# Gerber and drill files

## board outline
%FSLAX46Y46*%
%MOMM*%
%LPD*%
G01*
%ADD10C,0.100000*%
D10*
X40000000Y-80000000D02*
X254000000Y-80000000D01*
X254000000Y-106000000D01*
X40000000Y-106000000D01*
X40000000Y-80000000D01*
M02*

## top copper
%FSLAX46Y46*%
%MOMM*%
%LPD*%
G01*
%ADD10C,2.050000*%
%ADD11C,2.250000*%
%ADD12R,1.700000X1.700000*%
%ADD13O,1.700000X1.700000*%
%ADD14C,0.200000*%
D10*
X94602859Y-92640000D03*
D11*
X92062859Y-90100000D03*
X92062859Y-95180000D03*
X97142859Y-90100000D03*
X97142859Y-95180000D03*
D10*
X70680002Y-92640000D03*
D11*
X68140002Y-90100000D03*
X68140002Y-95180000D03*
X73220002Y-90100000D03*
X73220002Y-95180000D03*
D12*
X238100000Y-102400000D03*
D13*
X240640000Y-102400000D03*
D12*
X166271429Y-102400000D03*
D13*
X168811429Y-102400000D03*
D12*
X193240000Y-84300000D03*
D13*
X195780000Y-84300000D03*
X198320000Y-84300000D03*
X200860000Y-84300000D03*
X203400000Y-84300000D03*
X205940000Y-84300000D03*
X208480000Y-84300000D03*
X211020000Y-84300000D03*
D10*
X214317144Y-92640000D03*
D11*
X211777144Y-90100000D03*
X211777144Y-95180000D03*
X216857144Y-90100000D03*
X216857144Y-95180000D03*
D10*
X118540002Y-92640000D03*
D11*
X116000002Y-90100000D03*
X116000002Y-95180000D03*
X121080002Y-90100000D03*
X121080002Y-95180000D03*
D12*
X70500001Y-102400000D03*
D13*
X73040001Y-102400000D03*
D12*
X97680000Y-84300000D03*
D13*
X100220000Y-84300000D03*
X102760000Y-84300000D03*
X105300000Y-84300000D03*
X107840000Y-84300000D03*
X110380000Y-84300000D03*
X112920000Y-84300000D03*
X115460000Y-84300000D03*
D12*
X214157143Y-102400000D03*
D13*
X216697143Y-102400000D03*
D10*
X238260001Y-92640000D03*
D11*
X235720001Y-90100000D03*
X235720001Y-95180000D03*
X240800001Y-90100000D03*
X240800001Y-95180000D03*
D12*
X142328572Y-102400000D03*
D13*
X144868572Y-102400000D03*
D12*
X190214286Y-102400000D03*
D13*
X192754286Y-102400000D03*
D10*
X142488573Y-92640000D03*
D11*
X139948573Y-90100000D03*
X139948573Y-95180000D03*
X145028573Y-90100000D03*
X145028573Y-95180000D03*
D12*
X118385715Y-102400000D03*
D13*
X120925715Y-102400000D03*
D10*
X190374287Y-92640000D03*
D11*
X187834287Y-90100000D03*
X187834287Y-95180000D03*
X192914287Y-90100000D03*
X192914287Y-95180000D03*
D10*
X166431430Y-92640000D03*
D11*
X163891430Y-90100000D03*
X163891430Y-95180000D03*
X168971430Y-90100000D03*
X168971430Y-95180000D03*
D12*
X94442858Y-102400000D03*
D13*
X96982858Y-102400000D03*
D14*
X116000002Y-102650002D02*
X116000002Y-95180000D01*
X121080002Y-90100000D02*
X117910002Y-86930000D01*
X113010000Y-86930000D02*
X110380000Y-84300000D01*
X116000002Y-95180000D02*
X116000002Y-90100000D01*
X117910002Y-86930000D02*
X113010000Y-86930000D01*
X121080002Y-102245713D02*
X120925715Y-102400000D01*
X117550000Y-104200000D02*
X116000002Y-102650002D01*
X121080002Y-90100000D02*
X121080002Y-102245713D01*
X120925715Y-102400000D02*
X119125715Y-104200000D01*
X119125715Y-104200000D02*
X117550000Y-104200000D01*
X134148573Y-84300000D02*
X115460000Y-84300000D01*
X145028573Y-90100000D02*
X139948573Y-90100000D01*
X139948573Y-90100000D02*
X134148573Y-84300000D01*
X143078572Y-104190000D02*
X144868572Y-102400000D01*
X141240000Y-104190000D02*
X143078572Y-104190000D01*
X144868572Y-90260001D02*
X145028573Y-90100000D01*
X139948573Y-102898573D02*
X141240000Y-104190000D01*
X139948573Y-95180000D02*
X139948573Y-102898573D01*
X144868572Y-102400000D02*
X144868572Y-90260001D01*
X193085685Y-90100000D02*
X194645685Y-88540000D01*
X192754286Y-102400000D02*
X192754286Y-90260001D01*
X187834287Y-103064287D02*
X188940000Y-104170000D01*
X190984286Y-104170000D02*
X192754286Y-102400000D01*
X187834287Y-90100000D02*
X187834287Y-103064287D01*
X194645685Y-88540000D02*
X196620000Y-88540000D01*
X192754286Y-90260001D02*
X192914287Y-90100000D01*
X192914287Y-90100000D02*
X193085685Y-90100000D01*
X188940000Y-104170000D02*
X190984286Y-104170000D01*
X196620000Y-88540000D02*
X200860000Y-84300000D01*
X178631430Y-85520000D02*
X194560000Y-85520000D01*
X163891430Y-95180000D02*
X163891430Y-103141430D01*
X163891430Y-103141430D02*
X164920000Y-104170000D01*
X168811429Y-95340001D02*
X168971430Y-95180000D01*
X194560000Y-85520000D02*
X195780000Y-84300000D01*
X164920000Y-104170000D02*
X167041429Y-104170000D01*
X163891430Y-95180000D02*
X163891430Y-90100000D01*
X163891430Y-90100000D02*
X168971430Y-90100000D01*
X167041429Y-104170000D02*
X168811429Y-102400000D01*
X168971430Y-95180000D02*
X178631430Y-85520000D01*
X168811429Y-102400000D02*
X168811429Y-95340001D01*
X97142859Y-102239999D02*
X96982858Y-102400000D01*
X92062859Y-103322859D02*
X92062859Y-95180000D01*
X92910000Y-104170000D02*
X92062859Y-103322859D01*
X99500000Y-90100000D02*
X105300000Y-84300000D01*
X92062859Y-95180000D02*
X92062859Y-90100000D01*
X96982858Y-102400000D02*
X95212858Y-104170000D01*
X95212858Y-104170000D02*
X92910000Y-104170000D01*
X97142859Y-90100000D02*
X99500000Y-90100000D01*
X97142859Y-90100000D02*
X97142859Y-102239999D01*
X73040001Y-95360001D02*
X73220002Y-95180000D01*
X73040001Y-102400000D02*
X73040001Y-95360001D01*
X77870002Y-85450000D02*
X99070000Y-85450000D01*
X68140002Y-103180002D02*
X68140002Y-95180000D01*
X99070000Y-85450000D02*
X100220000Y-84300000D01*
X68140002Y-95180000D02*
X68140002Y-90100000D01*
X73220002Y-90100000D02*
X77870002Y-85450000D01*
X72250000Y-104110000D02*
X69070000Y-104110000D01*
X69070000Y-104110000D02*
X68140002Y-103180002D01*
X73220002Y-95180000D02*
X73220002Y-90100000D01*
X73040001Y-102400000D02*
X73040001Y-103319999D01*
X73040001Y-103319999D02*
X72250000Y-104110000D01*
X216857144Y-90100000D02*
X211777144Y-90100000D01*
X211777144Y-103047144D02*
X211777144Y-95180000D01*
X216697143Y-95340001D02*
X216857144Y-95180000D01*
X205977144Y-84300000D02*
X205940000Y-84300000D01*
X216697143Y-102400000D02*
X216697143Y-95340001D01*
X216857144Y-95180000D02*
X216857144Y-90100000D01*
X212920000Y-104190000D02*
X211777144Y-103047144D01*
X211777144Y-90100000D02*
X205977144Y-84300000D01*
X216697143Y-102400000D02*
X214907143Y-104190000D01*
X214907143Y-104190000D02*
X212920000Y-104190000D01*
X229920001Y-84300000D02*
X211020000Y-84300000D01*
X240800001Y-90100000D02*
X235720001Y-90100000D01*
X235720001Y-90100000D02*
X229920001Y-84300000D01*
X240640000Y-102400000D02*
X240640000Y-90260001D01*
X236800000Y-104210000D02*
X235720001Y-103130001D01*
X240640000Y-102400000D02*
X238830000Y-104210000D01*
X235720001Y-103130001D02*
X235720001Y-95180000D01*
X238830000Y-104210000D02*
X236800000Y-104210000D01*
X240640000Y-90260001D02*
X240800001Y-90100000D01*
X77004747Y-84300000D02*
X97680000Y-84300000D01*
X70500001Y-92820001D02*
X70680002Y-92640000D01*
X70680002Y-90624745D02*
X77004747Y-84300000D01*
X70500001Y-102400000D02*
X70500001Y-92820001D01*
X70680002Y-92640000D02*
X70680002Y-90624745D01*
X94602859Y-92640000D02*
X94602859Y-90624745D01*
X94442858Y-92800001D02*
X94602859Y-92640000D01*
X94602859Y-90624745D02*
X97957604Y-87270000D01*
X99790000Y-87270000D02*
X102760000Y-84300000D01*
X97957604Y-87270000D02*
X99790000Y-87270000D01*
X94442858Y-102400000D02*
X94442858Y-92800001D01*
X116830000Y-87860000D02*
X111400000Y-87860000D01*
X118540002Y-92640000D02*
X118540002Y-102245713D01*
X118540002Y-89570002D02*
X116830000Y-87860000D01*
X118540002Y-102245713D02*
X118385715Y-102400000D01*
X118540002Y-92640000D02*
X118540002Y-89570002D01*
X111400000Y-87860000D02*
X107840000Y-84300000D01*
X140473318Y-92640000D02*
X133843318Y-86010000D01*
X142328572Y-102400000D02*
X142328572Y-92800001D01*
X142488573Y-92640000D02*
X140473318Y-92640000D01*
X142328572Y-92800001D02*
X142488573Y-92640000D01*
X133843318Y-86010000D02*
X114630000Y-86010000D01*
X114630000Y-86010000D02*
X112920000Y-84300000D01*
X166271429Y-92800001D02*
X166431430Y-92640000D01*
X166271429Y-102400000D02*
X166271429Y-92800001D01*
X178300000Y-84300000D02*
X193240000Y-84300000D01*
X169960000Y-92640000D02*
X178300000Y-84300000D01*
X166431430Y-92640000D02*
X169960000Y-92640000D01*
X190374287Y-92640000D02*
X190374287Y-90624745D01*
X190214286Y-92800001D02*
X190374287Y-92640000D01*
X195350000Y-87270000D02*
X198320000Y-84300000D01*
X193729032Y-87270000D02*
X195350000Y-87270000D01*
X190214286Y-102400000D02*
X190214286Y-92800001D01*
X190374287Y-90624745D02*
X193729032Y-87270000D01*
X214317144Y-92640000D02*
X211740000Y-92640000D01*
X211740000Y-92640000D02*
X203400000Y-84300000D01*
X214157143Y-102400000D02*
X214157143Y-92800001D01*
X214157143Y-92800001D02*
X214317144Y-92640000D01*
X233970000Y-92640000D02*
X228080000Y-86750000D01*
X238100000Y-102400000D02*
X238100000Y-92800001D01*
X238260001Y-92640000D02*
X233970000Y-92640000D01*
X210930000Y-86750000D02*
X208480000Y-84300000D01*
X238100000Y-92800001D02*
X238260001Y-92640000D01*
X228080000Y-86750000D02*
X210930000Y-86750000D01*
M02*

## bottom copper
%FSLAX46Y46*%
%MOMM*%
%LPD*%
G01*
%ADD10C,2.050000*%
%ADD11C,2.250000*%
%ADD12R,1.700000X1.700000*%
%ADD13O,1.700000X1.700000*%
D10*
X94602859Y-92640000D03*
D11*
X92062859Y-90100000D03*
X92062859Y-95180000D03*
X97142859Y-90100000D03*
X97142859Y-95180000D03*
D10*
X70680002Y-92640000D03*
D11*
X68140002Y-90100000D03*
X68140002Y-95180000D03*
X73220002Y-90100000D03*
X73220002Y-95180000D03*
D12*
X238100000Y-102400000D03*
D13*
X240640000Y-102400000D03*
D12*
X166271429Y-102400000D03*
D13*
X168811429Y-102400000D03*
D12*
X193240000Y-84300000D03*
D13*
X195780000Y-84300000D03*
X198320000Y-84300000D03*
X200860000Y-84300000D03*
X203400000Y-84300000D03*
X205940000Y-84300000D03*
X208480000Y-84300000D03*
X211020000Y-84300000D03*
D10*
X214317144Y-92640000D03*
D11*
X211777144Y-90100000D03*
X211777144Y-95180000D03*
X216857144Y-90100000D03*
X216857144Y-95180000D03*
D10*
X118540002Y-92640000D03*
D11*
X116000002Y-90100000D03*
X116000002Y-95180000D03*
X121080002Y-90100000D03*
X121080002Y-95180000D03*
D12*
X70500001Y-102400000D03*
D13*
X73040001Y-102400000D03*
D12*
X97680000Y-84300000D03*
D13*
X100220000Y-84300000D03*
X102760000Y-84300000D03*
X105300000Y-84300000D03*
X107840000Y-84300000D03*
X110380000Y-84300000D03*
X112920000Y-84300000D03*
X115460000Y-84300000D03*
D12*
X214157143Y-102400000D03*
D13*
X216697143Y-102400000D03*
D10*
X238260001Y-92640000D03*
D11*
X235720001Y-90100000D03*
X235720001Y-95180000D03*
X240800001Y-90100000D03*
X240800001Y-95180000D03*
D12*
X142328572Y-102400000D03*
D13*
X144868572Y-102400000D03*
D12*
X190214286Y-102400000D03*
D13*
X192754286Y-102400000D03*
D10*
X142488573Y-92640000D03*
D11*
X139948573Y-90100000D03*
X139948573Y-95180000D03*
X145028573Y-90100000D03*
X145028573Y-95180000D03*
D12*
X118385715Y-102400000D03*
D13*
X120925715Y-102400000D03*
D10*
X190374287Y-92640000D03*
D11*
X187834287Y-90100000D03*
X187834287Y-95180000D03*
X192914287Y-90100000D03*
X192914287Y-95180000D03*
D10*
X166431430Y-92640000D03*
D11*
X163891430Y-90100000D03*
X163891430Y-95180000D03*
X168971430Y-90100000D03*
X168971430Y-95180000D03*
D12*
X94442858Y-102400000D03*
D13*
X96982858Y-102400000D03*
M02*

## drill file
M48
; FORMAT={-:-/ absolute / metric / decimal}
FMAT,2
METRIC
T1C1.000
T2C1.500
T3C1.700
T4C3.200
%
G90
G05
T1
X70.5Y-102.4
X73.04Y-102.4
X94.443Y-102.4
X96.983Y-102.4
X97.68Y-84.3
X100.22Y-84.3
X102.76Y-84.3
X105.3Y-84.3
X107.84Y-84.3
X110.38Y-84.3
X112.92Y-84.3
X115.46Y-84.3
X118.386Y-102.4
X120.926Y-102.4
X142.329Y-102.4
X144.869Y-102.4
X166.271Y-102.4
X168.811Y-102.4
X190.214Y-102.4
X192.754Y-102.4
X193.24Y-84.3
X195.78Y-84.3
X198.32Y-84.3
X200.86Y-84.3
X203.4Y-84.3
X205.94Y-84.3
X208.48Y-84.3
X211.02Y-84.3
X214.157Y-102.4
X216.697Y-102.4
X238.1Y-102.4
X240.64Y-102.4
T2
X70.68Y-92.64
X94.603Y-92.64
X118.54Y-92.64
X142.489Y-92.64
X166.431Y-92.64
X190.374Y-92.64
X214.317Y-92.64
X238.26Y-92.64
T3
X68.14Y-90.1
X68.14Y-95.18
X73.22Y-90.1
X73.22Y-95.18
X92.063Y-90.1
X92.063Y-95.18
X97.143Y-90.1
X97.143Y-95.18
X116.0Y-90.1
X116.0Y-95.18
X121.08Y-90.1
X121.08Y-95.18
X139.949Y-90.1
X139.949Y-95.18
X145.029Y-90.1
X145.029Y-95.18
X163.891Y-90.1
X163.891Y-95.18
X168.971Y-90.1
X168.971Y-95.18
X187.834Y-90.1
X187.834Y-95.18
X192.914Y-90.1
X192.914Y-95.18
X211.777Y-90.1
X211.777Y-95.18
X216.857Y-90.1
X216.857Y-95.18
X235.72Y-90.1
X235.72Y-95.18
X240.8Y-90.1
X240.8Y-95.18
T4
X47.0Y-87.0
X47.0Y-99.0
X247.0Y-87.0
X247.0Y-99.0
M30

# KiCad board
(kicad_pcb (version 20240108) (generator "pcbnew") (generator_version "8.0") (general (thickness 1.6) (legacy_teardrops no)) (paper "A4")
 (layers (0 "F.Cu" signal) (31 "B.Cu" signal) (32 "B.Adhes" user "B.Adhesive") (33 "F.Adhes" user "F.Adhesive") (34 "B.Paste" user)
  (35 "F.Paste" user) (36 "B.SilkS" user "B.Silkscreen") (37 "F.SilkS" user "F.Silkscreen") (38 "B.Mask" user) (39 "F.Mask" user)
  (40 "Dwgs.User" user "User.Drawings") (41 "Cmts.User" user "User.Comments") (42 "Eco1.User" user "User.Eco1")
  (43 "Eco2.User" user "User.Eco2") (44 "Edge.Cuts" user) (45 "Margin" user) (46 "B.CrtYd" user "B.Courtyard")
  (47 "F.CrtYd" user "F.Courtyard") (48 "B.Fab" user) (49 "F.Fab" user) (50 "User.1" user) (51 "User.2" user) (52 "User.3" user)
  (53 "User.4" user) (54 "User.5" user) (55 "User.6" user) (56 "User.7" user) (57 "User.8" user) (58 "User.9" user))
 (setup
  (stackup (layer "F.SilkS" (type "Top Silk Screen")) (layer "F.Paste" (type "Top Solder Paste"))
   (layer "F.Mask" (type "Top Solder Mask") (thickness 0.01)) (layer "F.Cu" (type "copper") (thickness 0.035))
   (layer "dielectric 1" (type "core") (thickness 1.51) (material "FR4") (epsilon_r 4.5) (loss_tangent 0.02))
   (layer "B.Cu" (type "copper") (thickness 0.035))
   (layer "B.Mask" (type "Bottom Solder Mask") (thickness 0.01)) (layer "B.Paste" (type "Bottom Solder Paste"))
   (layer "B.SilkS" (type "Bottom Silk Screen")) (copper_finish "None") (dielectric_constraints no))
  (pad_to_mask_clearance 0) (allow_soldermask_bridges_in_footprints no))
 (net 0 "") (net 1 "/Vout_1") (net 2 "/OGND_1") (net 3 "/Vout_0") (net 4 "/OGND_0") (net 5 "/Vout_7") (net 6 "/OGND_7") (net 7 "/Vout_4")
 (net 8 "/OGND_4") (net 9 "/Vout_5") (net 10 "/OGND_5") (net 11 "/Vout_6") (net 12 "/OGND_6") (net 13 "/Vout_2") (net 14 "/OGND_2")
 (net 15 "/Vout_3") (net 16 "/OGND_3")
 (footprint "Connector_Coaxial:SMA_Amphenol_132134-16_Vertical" (layer "F.Cu") (at 94.602859 92.64)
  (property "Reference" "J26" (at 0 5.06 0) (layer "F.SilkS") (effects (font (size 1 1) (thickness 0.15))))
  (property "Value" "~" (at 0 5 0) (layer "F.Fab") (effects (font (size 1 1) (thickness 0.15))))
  (pad "1" thru_hole circle (at 0 0) (size 2.05 2.05) (drill 1.5) (layers "*.Cu" "*.Mask") (remove_unused_layers no) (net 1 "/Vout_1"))
  (pad "2" thru_hole circle (at -2.54 -2.54) (size 2.25 2.25) (drill 1.7) (layers "*.Cu" "*.Mask") (remove_unused_layers no)
   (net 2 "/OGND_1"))
  (pad "2" thru_hole circle (at -2.54 2.54) (size 2.25 2.25) (drill 1.7) (layers "*.Cu" "*.Mask") (remove_unused_layers no)
   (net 2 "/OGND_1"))
  (pad "2" thru_hole circle (at 2.54 -2.54) (size 2.25 2.25) (drill 1.7) (layers "*.Cu" "*.Mask") (remove_unused_layers no)
   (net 2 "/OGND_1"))
  (pad "2" thru_hole circle (at 2.54 2.54) (size 2.25 2.25) (drill 1.7) (layers "*.Cu" "*.Mask") (remove_unused_layers no) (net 2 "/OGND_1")))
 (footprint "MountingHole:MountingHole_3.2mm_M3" (layer "F.Cu") (at 247 99)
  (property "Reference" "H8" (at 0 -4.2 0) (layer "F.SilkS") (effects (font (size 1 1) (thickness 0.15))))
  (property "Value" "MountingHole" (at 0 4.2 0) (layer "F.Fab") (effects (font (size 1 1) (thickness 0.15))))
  (pad "" np_thru_hole circle (at 0 0) (size 3.2 3.2) (drill 3.2) (layers "*.Cu" "*.Mask")))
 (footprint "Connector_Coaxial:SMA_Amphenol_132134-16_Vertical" (layer "F.Cu") (at 70.680002 92.64)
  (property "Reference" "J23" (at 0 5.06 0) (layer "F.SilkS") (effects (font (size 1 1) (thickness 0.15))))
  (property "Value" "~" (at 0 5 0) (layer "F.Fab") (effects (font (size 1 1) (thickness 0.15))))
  (pad "1" thru_hole circle (at 0 0) (size 2.05 2.05) (drill 1.5) (layers "*.Cu" "*.Mask") (remove_unused_layers no) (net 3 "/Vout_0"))
  (pad "2" thru_hole circle (at -2.54 -2.54) (size 2.25 2.25) (drill 1.7) (layers "*.Cu" "*.Mask") (remove_unused_layers no)
   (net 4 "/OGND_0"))
  (pad "2" thru_hole circle (at -2.54 2.54) (size 2.25 2.25) (drill 1.7) (layers "*.Cu" "*.Mask") (remove_unused_layers no)
   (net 4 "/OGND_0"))
  (pad "2" thru_hole circle (at 2.54 -2.54) (size 2.25 2.25) (drill 1.7) (layers "*.Cu" "*.Mask") (remove_unused_layers no)
   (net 4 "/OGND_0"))
  (pad "2" thru_hole circle (at 2.54 2.54) (size 2.25 2.25) (drill 1.7) (layers "*.Cu" "*.Mask") (remove_unused_layers no) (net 4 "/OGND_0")))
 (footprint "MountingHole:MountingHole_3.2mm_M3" (layer "F.Cu") (at 47 99)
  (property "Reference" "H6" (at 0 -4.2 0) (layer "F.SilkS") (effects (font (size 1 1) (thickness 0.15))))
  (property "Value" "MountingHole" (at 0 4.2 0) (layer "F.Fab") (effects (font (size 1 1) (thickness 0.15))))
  (pad "" np_thru_hole circle (at 0 0) (size 3.2 3.2) (drill 3.2) (layers "*.Cu" "*.Mask")))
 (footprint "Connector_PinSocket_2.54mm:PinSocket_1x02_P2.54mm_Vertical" (layer "F.Cu") (at 238.1 102.4 90)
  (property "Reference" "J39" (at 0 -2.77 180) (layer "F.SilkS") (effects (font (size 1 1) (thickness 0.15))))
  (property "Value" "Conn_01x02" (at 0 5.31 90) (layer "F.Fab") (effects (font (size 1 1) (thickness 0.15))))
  (pad "1" thru_hole rect (at 0 0 90) (size 1.7 1.7) (drill 1) (layers "*.Cu" "*.Mask") (remove_unused_layers no) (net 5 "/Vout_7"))
  (pad "2" thru_hole oval (at 0 2.54 90) (size 1.7 1.7) (drill 1) (layers "*.Cu" "*.Mask") (remove_unused_layers no) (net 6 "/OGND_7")))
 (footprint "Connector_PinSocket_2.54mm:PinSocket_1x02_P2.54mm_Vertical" (layer "F.Cu") (at 166.271429 102.4 90)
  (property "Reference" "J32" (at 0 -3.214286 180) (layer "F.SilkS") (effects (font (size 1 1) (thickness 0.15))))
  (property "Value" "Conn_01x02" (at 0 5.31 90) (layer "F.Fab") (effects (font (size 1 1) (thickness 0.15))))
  (pad "1" thru_hole rect (at 0 0 90) (size 1.7 1.7) (drill 1) (layers "*.Cu" "*.Mask") (remove_unused_layers no) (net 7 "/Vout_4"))
  (pad "2" thru_hole oval (at 0 2.54 90) (size 1.7 1.7) (drill 1) (layers "*.Cu" "*.Mask") (remove_unused_layers no) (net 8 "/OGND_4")))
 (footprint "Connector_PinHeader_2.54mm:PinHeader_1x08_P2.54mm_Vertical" (layer "F.Cu") (at 193.24 84.3 90)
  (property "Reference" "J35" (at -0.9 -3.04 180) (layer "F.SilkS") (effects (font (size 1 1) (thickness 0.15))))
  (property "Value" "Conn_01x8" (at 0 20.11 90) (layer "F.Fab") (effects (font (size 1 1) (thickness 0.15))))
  (pad "1" thru_hole rect (at 0 0 90) (size 1.7 1.7) (drill 1) (layers "*.Cu" "*.Mask") (remove_unused_layers no) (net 7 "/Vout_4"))
  (pad "2" thru_hole oval (at 0 2.54 90) (size 1.7 1.7) (drill 1) (layers "*.Cu" "*.Mask") (remove_unused_layers no) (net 8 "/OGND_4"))
  (pad "3" thru_hole oval (at 0 5.08 90) (size 1.7 1.7) (drill 1) (layers "*.Cu" "*.Mask") (remove_unused_layers no) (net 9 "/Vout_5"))
  (pad "4" thru_hole oval (at 0 7.62 90) (size 1.7 1.7) (drill 1) (layers "*.Cu" "*.Mask") (remove_unused_layers no) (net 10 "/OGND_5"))
  (pad "5" thru_hole oval (at 0 10.16 90) (size 1.7 1.7) (drill 1) (layers "*.Cu" "*.Mask") (remove_unused_layers no) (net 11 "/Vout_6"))
  (pad "6" thru_hole oval (at 0 12.7 90) (size 1.7 1.7) (drill 1) (layers "*.Cu" "*.Mask") (remove_unused_layers no) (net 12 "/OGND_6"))
  (pad "7" thru_hole oval (at 0 15.24 90) (size 1.7 1.7) (drill 1) (layers "*.Cu" "*.Mask") (remove_unused_layers no) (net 5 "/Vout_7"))
  (pad "8" thru_hole oval (at 0 17.78 90) (size 1.7 1.7) (drill 1) (layers "*.Cu" "*.Mask") (remove_unused_layers no) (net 6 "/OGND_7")))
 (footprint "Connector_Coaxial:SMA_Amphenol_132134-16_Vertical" (layer "F.Cu") (at 214.317144 92.64)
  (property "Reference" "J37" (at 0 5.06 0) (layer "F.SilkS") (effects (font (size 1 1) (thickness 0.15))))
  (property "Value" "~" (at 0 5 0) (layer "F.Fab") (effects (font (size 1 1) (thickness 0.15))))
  (pad "1" thru_hole circle (at 0 0) (size 2.05 2.05) (drill 1.5) (layers "*.Cu" "*.Mask") (remove_unused_layers no) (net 11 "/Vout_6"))
  (pad "2" thru_hole circle (at -2.54 -2.54) (size 2.25 2.25) (drill 1.7) (layers "*.Cu" "*.Mask") (remove_unused_layers no)
   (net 12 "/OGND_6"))
  (pad "2" thru_hole circle (at -2.54 2.54) (size 2.25 2.25) (drill 1.7) (layers "*.Cu" "*.Mask") (remove_unused_layers no)
   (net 12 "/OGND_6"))
  (pad "2" thru_hole circle (at 2.54 -2.54) (size 2.25 2.25) (drill 1.7) (layers "*.Cu" "*.Mask") (remove_unused_layers no)
   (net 12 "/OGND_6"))
  (pad "2" thru_hole circle (at 2.54 2.54) (size 2.25 2.25) (drill 1.7) (layers "*.Cu" "*.Mask") (remove_unused_layers no)
   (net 12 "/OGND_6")))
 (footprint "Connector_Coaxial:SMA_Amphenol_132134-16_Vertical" (layer "F.Cu") (at 118.540002 92.64)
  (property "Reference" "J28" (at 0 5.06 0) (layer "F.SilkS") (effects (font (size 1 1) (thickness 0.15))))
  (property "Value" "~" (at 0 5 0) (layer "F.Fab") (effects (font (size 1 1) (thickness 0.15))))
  (pad "1" thru_hole circle (at 0 0) (size 2.05 2.05) (drill 1.5) (layers "*.Cu" "*.Mask") (remove_unused_layers no) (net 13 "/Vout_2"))
  (pad "2" thru_hole circle (at -2.54 -2.54) (size 2.25 2.25) (drill 1.7) (layers "*.Cu" "*.Mask") (remove_unused_layers no)
   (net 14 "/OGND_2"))
  (pad "2" thru_hole circle (at -2.54 2.54) (size 2.25 2.25) (drill 1.7) (layers "*.Cu" "*.Mask") (remove_unused_layers no)
   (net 14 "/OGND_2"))
  (pad "2" thru_hole circle (at 2.54 -2.54) (size 2.25 2.25) (drill 1.7) (layers "*.Cu" "*.Mask") (remove_unused_layers no)
   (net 14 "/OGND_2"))
  (pad "2" thru_hole circle (at 2.54 2.54) (size 2.25 2.25) (drill 1.7) (layers "*.Cu" "*.Mask") (remove_unused_layers no)
   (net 14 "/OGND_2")))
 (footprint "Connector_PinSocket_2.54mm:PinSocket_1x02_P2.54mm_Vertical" (layer "F.Cu") (at 70.500001 102.4 90)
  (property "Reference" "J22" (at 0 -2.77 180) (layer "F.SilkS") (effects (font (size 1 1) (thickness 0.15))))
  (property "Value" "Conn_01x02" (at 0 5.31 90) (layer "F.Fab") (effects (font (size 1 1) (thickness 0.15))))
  (pad "1" thru_hole rect (at 0 0 90) (size 1.7 1.7) (drill 1) (layers "*.Cu" "*.Mask") (remove_unused_layers no) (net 3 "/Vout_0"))
  (pad "2" thru_hole oval (at 0 2.54 90) (size 1.7 1.7) (drill 1) (layers "*.Cu" "*.Mask") (remove_unused_layers no) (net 4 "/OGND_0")))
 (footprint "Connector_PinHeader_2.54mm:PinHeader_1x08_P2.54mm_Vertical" (layer "F.Cu") (at 97.68 84.3 90)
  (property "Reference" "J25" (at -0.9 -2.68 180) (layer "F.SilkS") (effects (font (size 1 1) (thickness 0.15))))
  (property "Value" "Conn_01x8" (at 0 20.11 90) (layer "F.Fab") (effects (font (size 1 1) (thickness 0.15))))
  (pad "1" thru_hole rect (at 0 0 90) (size 1.7 1.7) (drill 1) (layers "*.Cu" "*.Mask") (remove_unused_layers no) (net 3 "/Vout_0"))
  (pad "2" thru_hole oval (at 0 2.54 90) (size 1.7 1.7) (drill 1) (layers "*.Cu" "*.Mask") (remove_unused_layers no) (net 4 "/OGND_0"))
  (pad "3" thru_hole oval (at 0 5.08 90) (size 1.7 1.7) (drill 1) (layers "*.Cu" "*.Mask") (remove_unused_layers no) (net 1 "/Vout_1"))
  (pad "4" thru_hole oval (at 0 7.62 90) (size 1.7 1.7) (drill 1) (layers "*.Cu" "*.Mask") (remove_unused_layers no) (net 2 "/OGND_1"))
  (pad "5" thru_hole oval (at 0 10.16 90) (size 1.7 1.7) (drill 1) (layers "*.Cu" "*.Mask") (remove_unused_layers no) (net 13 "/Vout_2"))
  (pad "6" thru_hole oval (at 0 12.7 90) (size 1.7 1.7) (drill 1) (layers "*.Cu" "*.Mask") (remove_unused_layers no) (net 14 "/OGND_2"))
  (pad "7" thru_hole oval (at 0 15.24 90) (size 1.7 1.7) (drill 1) (layers "*.Cu" "*.Mask") (remove_unused_layers no) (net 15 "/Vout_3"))
  (pad "8" thru_hole oval (at 0 17.78 90) (size 1.7 1.7) (drill 1) (layers "*.Cu" "*.Mask") (remove_unused_layers no) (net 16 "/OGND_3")))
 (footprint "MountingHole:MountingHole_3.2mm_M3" (layer "F.Cu") (at 247 87)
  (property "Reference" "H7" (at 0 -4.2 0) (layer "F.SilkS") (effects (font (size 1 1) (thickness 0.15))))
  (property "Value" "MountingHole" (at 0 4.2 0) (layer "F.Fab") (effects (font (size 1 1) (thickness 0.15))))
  (pad "" np_thru_hole circle (at 0 0) (size 3.2 3.2) (drill 3.2) (layers "*.Cu" "*.Mask")))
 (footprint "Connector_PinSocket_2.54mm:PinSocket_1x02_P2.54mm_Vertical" (layer "F.Cu") (at 214.157143 102.4 90)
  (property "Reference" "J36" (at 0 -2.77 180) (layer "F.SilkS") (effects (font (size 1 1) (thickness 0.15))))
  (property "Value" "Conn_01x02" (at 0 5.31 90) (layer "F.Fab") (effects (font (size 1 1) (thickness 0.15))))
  (pad "1" thru_hole rect (at 0 0 90) (size 1.7 1.7) (drill 1) (layers "*.Cu" "*.Mask") (remove_unused_layers no) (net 11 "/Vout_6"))
  (pad "2" thru_hole oval (at 0 2.54 90) (size 1.7 1.7) (drill 1) (layers "*.Cu" "*.Mask") (remove_unused_layers no) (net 12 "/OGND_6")))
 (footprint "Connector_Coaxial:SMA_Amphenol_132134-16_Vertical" (layer "F.Cu") (at 238.260001 92.64)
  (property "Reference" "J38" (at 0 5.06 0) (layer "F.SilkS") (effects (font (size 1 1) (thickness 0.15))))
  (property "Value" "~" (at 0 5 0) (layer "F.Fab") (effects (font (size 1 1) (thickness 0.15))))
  (pad "1" thru_hole circle (at 0 0) (size 2.05 2.05) (drill 1.5) (layers "*.Cu" "*.Mask") (remove_unused_layers no) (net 5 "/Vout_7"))
  (pad "2" thru_hole circle (at -2.54 -2.54) (size 2.25 2.25) (drill 1.7) (layers "*.Cu" "*.Mask") (remove_unused_layers no)
   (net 6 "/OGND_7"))
  (pad "2" thru_hole circle (at -2.54 2.54) (size 2.25 2.25) (drill 1.7) (layers "*.Cu" "*.Mask") (remove_unused_layers no)
   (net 6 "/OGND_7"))
  (pad "2" thru_hole circle (at 2.54 -2.54) (size 2.25 2.25) (drill 1.7) (layers "*.Cu" "*.Mask") (remove_unused_layers no)
   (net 6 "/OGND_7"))
  (pad "2" thru_hole circle (at 2.54 2.54) (size 2.25 2.25) (drill 1.7) (layers "*.Cu" "*.Mask") (remove_unused_layers no) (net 6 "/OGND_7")))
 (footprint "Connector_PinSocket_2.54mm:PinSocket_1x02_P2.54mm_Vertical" (layer "F.Cu") (at 142.328572 102.4 90)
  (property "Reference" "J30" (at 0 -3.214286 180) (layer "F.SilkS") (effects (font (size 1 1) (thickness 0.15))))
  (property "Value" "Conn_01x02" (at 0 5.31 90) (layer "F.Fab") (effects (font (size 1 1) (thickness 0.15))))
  (pad "1" thru_hole rect (at 0 0 90) (size 1.7 1.7) (drill 1) (layers "*.Cu" "*.Mask") (remove_unused_layers no) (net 15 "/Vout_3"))
  (pad "2" thru_hole oval (at 0 2.54 90) (size 1.7 1.7) (drill 1) (layers "*.Cu" "*.Mask") (remove_unused_layers no) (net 16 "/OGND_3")))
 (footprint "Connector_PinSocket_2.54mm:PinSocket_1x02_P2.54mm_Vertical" (layer "F.Cu") (at 190.214286 102.4 90)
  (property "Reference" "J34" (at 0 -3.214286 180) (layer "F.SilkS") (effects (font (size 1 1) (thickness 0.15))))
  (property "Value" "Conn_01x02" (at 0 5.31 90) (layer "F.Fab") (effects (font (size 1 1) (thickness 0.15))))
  (pad "1" thru_hole rect (at 0 0 90) (size 1.7 1.7) (drill 1) (layers "*.Cu" "*.Mask") (remove_unused_layers no) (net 9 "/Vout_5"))
  (pad "2" thru_hole oval (at 0 2.54 90) (size 1.7 1.7) (drill 1) (layers "*.Cu" "*.Mask") (remove_unused_layers no) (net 10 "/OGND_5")))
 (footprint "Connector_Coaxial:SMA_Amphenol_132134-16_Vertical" (layer "F.Cu") (at 142.488573 92.64)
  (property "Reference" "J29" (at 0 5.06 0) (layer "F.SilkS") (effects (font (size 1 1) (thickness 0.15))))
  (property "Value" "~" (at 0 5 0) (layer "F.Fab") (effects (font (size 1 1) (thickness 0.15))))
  (pad "1" thru_hole circle (at 0 0) (size 2.05 2.05) (drill 1.5) (layers "*.Cu" "*.Mask") (remove_unused_layers no) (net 15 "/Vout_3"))
  (pad "2" thru_hole circle (at -2.54 -2.54) (size 2.25 2.25) (drill 1.7) (layers "*.Cu" "*.Mask") (remove_unused_layers no)
   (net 16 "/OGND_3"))
  (pad "2" thru_hole circle (at -2.54 2.54) (size 2.25 2.25) (drill 1.7) (layers "*.Cu" "*.Mask") (remove_unused_layers no)
   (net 16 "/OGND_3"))
  (pad "2" thru_hole circle (at 2.54 -2.54) (size 2.25 2.25) (drill 1.7) (layers "*.Cu" "*.Mask") (remove_unused_layers no)
   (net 16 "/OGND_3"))
  (pad "2" thru_hole circle (at 2.54 2.54) (size 2.25 2.25) (drill 1.7) (layers "*.Cu" "*.Mask") (remove_unused_layers no)
   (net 16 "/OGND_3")))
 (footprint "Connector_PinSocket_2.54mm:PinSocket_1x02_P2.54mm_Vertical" (layer "F.Cu") (at 118.385715 102.4 90)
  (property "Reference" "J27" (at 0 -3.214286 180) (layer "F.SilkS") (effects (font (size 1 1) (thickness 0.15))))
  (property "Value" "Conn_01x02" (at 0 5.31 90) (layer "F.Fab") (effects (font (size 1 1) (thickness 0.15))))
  (pad "1" thru_hole rect (at 0 0 90) (size 1.7 1.7) (drill 1) (layers "*.Cu" "*.Mask") (remove_unused_layers no) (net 13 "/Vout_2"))
  (pad "2" thru_hole oval (at 0 2.54 90) (size 1.7 1.7) (drill 1) (layers "*.Cu" "*.Mask") (remove_unused_layers no) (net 14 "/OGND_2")))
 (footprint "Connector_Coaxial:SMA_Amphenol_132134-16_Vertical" (layer "F.Cu") (at 190.374287 92.64)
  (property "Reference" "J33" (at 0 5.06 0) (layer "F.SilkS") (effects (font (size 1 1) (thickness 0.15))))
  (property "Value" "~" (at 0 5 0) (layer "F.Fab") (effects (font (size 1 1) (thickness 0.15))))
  (pad "1" thru_hole circle (at 0 0) (size 2.05 2.05) (drill 1.5) (layers "*.Cu" "*.Mask") (remove_unused_layers no) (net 9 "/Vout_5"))
  (pad "2" thru_hole circle (at -2.54 -2.54) (size 2.25 2.25) (drill 1.7) (layers "*.Cu" "*.Mask") (remove_unused_layers no)
   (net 10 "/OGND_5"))
  (pad "2" thru_hole circle (at -2.54 2.54) (size 2.25 2.25) (drill 1.7) (layers "*.Cu" "*.Mask") (remove_unused_layers no)
   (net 10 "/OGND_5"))
  (pad "2" thru_hole circle (at 2.54 -2.54) (size 2.25 2.25) (drill 1.7) (layers "*.Cu" "*.Mask") (remove_unused_layers no)
   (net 10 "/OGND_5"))
  (pad "2" thru_hole circle (at 2.54 2.54) (size 2.25 2.25) (drill 1.7) (layers "*.Cu" "*.Mask") (remove_unused_layers no)
   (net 10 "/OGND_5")))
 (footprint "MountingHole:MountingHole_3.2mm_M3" (layer "F.Cu") (at 47 87)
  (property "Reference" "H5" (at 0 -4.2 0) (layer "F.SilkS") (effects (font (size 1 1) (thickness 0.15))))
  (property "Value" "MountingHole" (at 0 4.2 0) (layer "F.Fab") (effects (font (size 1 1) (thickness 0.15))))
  (pad "" np_thru_hole circle (at 0 0) (size 3.2 3.2) (drill 3.2) (layers "*.Cu" "*.Mask")))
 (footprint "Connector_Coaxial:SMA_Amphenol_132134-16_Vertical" (layer "F.Cu") (at 166.43143 92.64)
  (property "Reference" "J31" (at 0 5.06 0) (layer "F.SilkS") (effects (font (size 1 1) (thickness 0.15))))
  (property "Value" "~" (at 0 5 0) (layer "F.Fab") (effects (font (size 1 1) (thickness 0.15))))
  (pad "1" thru_hole circle (at 0 0) (size 2.05 2.05) (drill 1.5) (layers "*.Cu" "*.Mask") (remove_unused_layers no) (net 7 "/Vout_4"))
  (pad "2" thru_hole circle (at -2.54 -2.54) (size 2.25 2.25) (drill 1.7) (layers "*.Cu" "*.Mask") (remove_unused_layers no)
   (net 8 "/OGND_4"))
  (pad "2" thru_hole circle (at -2.54 2.54) (size 2.25 2.25) (drill 1.7) (layers "*.Cu" "*.Mask") (remove_unused_layers no)
   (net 8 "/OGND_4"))
  (pad "2" thru_hole circle (at 2.54 -2.54) (size 2.25 2.25) (drill 1.7) (layers "*.Cu" "*.Mask") (remove_unused_layers no)
   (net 8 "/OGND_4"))
  (pad "2" thru_hole circle (at 2.54 2.54) (size 2.25 2.25) (drill 1.7) (layers "*.Cu" "*.Mask") (remove_unused_layers no) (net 8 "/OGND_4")))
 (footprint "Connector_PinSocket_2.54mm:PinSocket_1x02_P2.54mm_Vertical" (layer "F.Cu") (at 94.442858 102.4 90)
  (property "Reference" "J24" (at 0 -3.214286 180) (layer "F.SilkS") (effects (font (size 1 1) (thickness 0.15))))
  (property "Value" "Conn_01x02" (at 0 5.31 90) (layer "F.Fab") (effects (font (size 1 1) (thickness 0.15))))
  (pad "1" thru_hole rect (at 0 0 90) (size 1.7 1.7) (drill 1) (layers "*.Cu" "*.Mask") (remove_unused_layers no) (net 1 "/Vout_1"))
  (pad "2" thru_hole oval (at 0 2.54 90) (size 1.7 1.7) (drill 1) (layers "*.Cu" "*.Mask") (remove_unused_layers no) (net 2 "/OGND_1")))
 (gr_rect (start 40 80) (end 254 106) (stroke (width 0.1) (type default)) (fill none) (layer "Edge.Cuts"))
 (segment (start 116.000002 102.650002) (end 116.000002 95.18) (width 0.2) (layer "F.Cu") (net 14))
 (segment (start 121.080002 90.1) (end 117.910002 86.93) (width 0.2) (layer "F.Cu") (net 14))
 (segment (start 113.01 86.93) (end 110.38 84.3) (width 0.2) (layer "F.Cu") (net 14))
 (segment (start 116.000002 95.18) (end 116.000002 90.1) (width 0.2) (layer "F.Cu") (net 14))
 (segment (start 117.910002 86.93) (end 113.01 86.93) (width 0.2) (layer "F.Cu") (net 14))
 (segment (start 121.080002 102.245713) (end 120.925715 102.4) (width 0.2) (layer "F.Cu") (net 14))
 (segment (start 117.55 104.2) (end 116.000002 102.650002) (width 0.2) (layer "F.Cu") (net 14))
 (segment (start 121.080002 90.1) (end 121.080002 102.245713) (width 0.2) (layer "F.Cu") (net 14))
 (segment (start 120.925715 102.4) (end 119.125715 104.2) (width 0.2) (layer "F.Cu") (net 14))
 (segment (start 119.125715 104.2) (end 117.55 104.2) (width 0.2) (layer "F.Cu") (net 14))
 (segment (start 134.148573 84.3) (end 115.46 84.3) (width 0.2) (layer "F.Cu") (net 16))
 (segment (start 145.028573 90.1) (end 139.948573 90.1) (width 0.2) (layer "F.Cu") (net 16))
 (segment (start 139.948573 90.1) (end 134.148573 84.3) (width 0.2) (layer "F.Cu") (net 16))
 (segment (start 143.078572 104.19) (end 144.868572 102.4) (width 0.2) (layer "F.Cu") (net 16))
 (segment (start 141.24 104.19) (end 143.078572 104.19) (width 0.2) (layer "F.Cu") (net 16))
 (segment (start 144.868572 90.260001) (end 145.028573 90.1) (width 0.2) (layer "F.Cu") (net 16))
 (segment (start 139.948573 102.898573) (end 141.24 104.19) (width 0.2) (layer "F.Cu") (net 16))
 (segment (start 139.948573 95.18) (end 139.948573 102.898573) (width 0.2) (layer "F.Cu") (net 16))
 (segment (start 144.868572 102.4) (end 144.868572 90.260001) (width 0.2) (layer "F.Cu") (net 16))
 (segment (start 193.085685 90.1) (end 194.645685 88.54) (width 0.2) (layer "F.Cu") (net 10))
 (segment (start 192.754286 102.4) (end 192.754286 90.260001) (width 0.2) (layer "F.Cu") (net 10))
 (segment (start 187.834287 103.064287) (end 188.94 104.17) (width 0.2) (layer "F.Cu") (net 10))
 (segment (start 190.984286 104.17) (end 192.754286 102.4) (width 0.2) (layer "F.Cu") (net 10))
 (segment (start 187.834287 90.1) (end 187.834287 103.064287) (width 0.2) (layer "F.Cu") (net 10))
 (segment (start 194.645685 88.54) (end 196.62 88.54) (width 0.2) (layer "F.Cu") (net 10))
 (segment (start 192.754286 90.260001) (end 192.914287 90.1) (width 0.2) (layer "F.Cu") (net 10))
 (segment (start 192.914287 90.1) (end 193.085685 90.1) (width 0.2) (layer "F.Cu") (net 10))
 (segment (start 188.94 104.17) (end 190.984286 104.17) (width 0.2) (layer "F.Cu") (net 10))
 (segment (start 196.62 88.54) (end 200.86 84.3) (width 0.2) (layer "F.Cu") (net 10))
 (segment (start 178.63143 85.52) (end 194.56 85.52) (width 0.2) (layer "F.Cu") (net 8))
 (segment (start 163.89143 95.18) (end 163.89143 103.14143) (width 0.2) (layer "F.Cu") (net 8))
 (segment (start 163.89143 103.14143) (end 164.92 104.17) (width 0.2) (layer "F.Cu") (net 8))
 (segment (start 168.811429 95.340001) (end 168.97143 95.18) (width 0.2) (layer "F.Cu") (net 8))
 (segment (start 194.56 85.52) (end 195.78 84.3) (width 0.2) (layer "F.Cu") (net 8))
 (segment (start 164.92 104.17) (end 167.041429 104.17) (width 0.2) (layer "F.Cu") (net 8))
 (segment (start 163.89143 95.18) (end 163.89143 90.1) (width 0.2) (layer "F.Cu") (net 8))
 (segment (start 163.89143 90.1) (end 168.97143 90.1) (width 0.2) (layer "F.Cu") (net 8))
 (segment (start 167.041429 104.17) (end 168.811429 102.4) (width 0.2) (layer "F.Cu") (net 8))
 (segment (start 168.97143 95.18) (end 178.63143 85.52) (width 0.2) (layer "F.Cu") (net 8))
 (segment (start 168.811429 102.4) (end 168.811429 95.340001) (width 0.2) (layer "F.Cu") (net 8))
 (segment (start 97.142859 102.239999) (end 96.982858 102.4) (width 0.2) (layer "F.Cu") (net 2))
 (segment (start 92.062859 103.322859) (end 92.062859 95.18) (width 0.2) (layer "F.Cu") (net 2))
 (segment (start 92.91 104.17) (end 92.062859 103.322859) (width 0.2) (layer "F.Cu") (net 2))
 (segment (start 99.5 90.1) (end 105.3 84.3) (width 0.2) (layer "F.Cu") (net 2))
 (segment (start 92.062859 95.18) (end 92.062859 90.1) (width 0.2) (layer "F.Cu") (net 2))
 (segment (start 96.982858 102.4) (end 95.212858 104.17) (width 0.2) (layer "F.Cu") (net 2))
 (segment (start 95.212858 104.17) (end 92.91 104.17) (width 0.2) (layer "F.Cu") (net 2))
 (segment (start 97.142859 90.1) (end 99.5 90.1) (width 0.2) (layer "F.Cu") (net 2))
 (segment (start 97.142859 90.1) (end 97.142859 102.239999) (width 0.2) (layer "F.Cu") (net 2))
 (segment (start 73.040001 95.360001) (end 73.220002 95.18) (width 0.2) (layer "F.Cu") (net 4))
 (segment (start 73.040001 102.4) (end 73.040001 95.360001) (width 0.2) (layer "F.Cu") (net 4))
 (segment (start 77.870002 85.45) (end 99.07 85.45) (width 0.2) (layer "F.Cu") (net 4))
 (segment (start 68.140002 103.180002) (end 68.140002 95.18) (width 0.2) (layer "F.Cu") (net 4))
 (segment (start 99.07 85.45) (end 100.22 84.3) (width 0.2) (layer "F.Cu") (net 4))
 (segment (start 68.140002 95.18) (end 68.140002 90.1) (width 0.2) (layer "F.Cu") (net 4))
 (segment (start 73.220002 90.1) (end 77.870002 85.45) (width 0.2) (layer "F.Cu") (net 4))
 (segment (start 72.25 104.11) (end 69.07 104.11) (width 0.2) (layer "F.Cu") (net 4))
 (segment (start 69.07 104.11) (end 68.140002 103.180002) (width 0.2) (layer "F.Cu") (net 4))
 (segment (start 73.220002 95.18) (end 73.220002 90.1) (width 0.2) (layer "F.Cu") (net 4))
 (segment (start 73.040001 102.4) (end 73.040001 103.319999) (width 0.2) (layer "F.Cu") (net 4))
 (segment (start 73.040001 103.319999) (end 72.25 104.11) (width 0.2) (layer "F.Cu") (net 4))
 (segment (start 216.857144 90.1) (end 211.777144 90.1) (width 0.2) (layer "F.Cu") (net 12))
 (segment (start 211.777144 103.047144) (end 211.777144 95.18) (width 0.2) (layer "F.Cu") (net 12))
 (segment (start 216.697143 95.340001) (end 216.857144 95.18) (width 0.2) (layer "F.Cu") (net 12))
 (segment (start 205.977144 84.3) (end 205.94 84.3) (width 0.2) (layer "F.Cu") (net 12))
 (segment (start 216.697143 102.4) (end 216.697143 95.340001) (width 0.2) (layer "F.Cu") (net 12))
 (segment (start 216.857144 95.18) (end 216.857144 90.1) (width 0.2) (layer "F.Cu") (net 12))
 (segment (start 212.92 104.19) (end 211.777144 103.047144) (width 0.2) (layer "F.Cu") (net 12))
 (segment (start 211.777144 90.1) (end 205.977144 84.3) (width 0.2) (layer "F.Cu") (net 12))
 (segment (start 216.697143 102.4) (end 214.907143 104.19) (width 0.2) (layer "F.Cu") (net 12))
 (segment (start 214.907143 104.19) (end 212.92 104.19) (width 0.2) (layer "F.Cu") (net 12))
 (segment (start 229.920001 84.3) (end 211.02 84.3) (width 0.2) (layer "F.Cu") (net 6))
 (segment (start 240.800001 90.1) (end 235.720001 90.1) (width 0.2) (layer "F.Cu") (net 6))
 (segment (start 235.720001 90.1) (end 229.920001 84.3) (width 0.2) (layer "F.Cu") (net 6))
 (segment (start 240.64 102.4) (end 240.64 90.260001) (width 0.2) (layer "F.Cu") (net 6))
 (segment (start 236.8 104.21) (end 235.720001 103.130001) (width 0.2) (layer "F.Cu") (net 6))
 (segment (start 240.64 102.4) (end 238.83 104.21) (width 0.2) (layer "F.Cu") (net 6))
 (segment (start 235.720001 103.130001) (end 235.720001 95.18) (width 0.2) (layer "F.Cu") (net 6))
 (segment (start 238.83 104.21) (end 236.8 104.21) (width 0.2) (layer "F.Cu") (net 6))
 (segment (start 240.64 90.260001) (end 240.800001 90.1) (width 0.2) (layer "F.Cu") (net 6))
 (segment (start 77.004747 84.3) (end 97.68 84.3) (width 0.2) (layer "F.Cu") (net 3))
 (segment (start 70.500001 92.820001) (end 70.680002 92.64) (width 0.2) (layer "F.Cu") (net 3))
 (segment (start 70.680002 90.624745) (end 77.004747 84.3) (width 0.2) (layer "F.Cu") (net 3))
 (segment (start 70.500001 102.4) (end 70.500001 92.820001) (width 0.2) (layer "F.Cu") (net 3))
 (segment (start 70.680002 92.64) (end 70.680002 90.624745) (width 0.2) (layer "F.Cu") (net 3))
 (segment (start 94.602859 92.64) (end 94.602859 90.624745) (width 0.2) (layer "F.Cu") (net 1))
 (segment (start 94.442858 92.800001) (end 94.602859 92.64) (width 0.2) (layer "F.Cu") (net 1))
 (segment (start 94.602859 90.624745) (end 97.957604 87.27) (width 0.2) (layer "F.Cu") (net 1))
 (segment (start 99.79 87.27) (end 102.76 84.3) (width 0.2) (layer "F.Cu") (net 1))
 (segment (start 97.957604 87.27) (end 99.79 87.27) (width 0.2) (layer "F.Cu") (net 1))
 (segment (start 94.442858 102.4) (end 94.442858 92.800001) (width 0.2) (layer "F.Cu") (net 1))
 (segment (start 116.83 87.86) (end 111.4 87.86) (width 0.2) (layer "F.Cu") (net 13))
 (segment (start 118.540002 92.64) (end 118.540002 102.245713) (width 0.2) (layer "F.Cu") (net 13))
 (segment (start 118.540002 89.570002) (end 116.83 87.86) (width 0.2) (layer "F.Cu") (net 13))
 (segment (start 118.540002 102.245713) (end 118.385715 102.4) (width 0.2) (layer "F.Cu") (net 13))
 (segment (start 118.540002 92.64) (end 118.540002 89.570002) (width 0.2) (layer "F.Cu") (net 13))
 (segment (start 111.4 87.86) (end 107.84 84.3) (width 0.2) (layer "F.Cu") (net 13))
 (segment (start 140.473318 92.64) (end 133.843318 86.01) (width 0.2) (layer "F.Cu") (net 15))
 (segment (start 142.328572 102.4) (end 142.328572 92.800001) (width 0.2) (layer "F.Cu") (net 15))
 (segment (start 142.488573 92.64) (end 140.473318 92.64) (width 0.2) (layer "F.Cu") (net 15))
 (segment (start 142.328572 92.800001) (end 142.488573 92.64) (width 0.2) (layer "F.Cu") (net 15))
 (segment (start 133.843318 86.01) (end 114.63 86.01) (width 0.2) (layer "F.Cu") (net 15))
 (segment (start 114.63 86.01) (end 112.92 84.3) (width 0.2) (layer "F.Cu") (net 15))
 (segment (start 166.271429 92.800001) (end 166.43143 92.64) (width 0.2) (layer "F.Cu") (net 7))
 (segment (start 166.271429 102.4) (end 166.271429 92.800001) (width 0.2) (layer "F.Cu") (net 7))
 (segment (start 178.3 84.3) (end 193.24 84.3) (width 0.2) (layer "F.Cu") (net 7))
 (segment (start 169.96 92.64) (end 178.3 84.3) (width 0.2) (layer "F.Cu") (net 7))
 (segment (start 166.43143 92.64) (end 169.96 92.64) (width 0.2) (layer "F.Cu") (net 7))
 (segment (start 190.374287 92.64) (end 190.374287 90.624745) (width 0.2) (layer "F.Cu") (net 9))
 (segment (start 190.214286 92.800001) (end 190.374287 92.64) (width 0.2) (layer "F.Cu") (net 9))
 (segment (start 195.35 87.27) (end 198.32 84.3) (width 0.2) (layer "F.Cu") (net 9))
 (segment (start 193.729032 87.27) (end 195.35 87.27) (width 0.2) (layer "F.Cu") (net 9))
 (segment (start 190.214286 102.4) (end 190.214286 92.800001) (width 0.2) (layer "F.Cu") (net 9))
 (segment (start 190.374287 90.624745) (end 193.729032 87.27) (width 0.2) (layer "F.Cu") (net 9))
 (segment (start 214.317144 92.64) (end 211.74 92.64) (width 0.2) (layer "F.Cu") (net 11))
 (segment (start 211.74 92.64) (end 203.4 84.3) (width 0.2) (layer "F.Cu") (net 11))
 (segment (start 214.157143 102.4) (end 214.157143 92.800001) (width 0.2) (layer "F.Cu") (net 11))
 (segment (start 214.157143 92.800001) (end 214.317144 92.64) (width 0.2) (layer "F.Cu") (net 11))
 (segment (start 233.97 92.64) (end 228.08 86.75) (width 0.2) (layer "F.Cu") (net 5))
 (segment (start 238.1 102.4) (end 238.1 92.800001) (width 0.2) (layer "F.Cu") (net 5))
 (segment (start 238.260001 92.64) (end 233.97 92.64) (width 0.2) (layer "F.Cu") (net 5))
 (segment (start 210.93 86.75) (end 208.48 84.3) (width 0.2) (layer "F.Cu") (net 5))
 (segment (start 238.1 92.800001) (end 238.260001 92.64) (width 0.2) (layer "F.Cu") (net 5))
 (segment (start 228.08 86.75) (end 210.93 86.75) (width 0.2) (layer "F.Cu") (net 5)))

